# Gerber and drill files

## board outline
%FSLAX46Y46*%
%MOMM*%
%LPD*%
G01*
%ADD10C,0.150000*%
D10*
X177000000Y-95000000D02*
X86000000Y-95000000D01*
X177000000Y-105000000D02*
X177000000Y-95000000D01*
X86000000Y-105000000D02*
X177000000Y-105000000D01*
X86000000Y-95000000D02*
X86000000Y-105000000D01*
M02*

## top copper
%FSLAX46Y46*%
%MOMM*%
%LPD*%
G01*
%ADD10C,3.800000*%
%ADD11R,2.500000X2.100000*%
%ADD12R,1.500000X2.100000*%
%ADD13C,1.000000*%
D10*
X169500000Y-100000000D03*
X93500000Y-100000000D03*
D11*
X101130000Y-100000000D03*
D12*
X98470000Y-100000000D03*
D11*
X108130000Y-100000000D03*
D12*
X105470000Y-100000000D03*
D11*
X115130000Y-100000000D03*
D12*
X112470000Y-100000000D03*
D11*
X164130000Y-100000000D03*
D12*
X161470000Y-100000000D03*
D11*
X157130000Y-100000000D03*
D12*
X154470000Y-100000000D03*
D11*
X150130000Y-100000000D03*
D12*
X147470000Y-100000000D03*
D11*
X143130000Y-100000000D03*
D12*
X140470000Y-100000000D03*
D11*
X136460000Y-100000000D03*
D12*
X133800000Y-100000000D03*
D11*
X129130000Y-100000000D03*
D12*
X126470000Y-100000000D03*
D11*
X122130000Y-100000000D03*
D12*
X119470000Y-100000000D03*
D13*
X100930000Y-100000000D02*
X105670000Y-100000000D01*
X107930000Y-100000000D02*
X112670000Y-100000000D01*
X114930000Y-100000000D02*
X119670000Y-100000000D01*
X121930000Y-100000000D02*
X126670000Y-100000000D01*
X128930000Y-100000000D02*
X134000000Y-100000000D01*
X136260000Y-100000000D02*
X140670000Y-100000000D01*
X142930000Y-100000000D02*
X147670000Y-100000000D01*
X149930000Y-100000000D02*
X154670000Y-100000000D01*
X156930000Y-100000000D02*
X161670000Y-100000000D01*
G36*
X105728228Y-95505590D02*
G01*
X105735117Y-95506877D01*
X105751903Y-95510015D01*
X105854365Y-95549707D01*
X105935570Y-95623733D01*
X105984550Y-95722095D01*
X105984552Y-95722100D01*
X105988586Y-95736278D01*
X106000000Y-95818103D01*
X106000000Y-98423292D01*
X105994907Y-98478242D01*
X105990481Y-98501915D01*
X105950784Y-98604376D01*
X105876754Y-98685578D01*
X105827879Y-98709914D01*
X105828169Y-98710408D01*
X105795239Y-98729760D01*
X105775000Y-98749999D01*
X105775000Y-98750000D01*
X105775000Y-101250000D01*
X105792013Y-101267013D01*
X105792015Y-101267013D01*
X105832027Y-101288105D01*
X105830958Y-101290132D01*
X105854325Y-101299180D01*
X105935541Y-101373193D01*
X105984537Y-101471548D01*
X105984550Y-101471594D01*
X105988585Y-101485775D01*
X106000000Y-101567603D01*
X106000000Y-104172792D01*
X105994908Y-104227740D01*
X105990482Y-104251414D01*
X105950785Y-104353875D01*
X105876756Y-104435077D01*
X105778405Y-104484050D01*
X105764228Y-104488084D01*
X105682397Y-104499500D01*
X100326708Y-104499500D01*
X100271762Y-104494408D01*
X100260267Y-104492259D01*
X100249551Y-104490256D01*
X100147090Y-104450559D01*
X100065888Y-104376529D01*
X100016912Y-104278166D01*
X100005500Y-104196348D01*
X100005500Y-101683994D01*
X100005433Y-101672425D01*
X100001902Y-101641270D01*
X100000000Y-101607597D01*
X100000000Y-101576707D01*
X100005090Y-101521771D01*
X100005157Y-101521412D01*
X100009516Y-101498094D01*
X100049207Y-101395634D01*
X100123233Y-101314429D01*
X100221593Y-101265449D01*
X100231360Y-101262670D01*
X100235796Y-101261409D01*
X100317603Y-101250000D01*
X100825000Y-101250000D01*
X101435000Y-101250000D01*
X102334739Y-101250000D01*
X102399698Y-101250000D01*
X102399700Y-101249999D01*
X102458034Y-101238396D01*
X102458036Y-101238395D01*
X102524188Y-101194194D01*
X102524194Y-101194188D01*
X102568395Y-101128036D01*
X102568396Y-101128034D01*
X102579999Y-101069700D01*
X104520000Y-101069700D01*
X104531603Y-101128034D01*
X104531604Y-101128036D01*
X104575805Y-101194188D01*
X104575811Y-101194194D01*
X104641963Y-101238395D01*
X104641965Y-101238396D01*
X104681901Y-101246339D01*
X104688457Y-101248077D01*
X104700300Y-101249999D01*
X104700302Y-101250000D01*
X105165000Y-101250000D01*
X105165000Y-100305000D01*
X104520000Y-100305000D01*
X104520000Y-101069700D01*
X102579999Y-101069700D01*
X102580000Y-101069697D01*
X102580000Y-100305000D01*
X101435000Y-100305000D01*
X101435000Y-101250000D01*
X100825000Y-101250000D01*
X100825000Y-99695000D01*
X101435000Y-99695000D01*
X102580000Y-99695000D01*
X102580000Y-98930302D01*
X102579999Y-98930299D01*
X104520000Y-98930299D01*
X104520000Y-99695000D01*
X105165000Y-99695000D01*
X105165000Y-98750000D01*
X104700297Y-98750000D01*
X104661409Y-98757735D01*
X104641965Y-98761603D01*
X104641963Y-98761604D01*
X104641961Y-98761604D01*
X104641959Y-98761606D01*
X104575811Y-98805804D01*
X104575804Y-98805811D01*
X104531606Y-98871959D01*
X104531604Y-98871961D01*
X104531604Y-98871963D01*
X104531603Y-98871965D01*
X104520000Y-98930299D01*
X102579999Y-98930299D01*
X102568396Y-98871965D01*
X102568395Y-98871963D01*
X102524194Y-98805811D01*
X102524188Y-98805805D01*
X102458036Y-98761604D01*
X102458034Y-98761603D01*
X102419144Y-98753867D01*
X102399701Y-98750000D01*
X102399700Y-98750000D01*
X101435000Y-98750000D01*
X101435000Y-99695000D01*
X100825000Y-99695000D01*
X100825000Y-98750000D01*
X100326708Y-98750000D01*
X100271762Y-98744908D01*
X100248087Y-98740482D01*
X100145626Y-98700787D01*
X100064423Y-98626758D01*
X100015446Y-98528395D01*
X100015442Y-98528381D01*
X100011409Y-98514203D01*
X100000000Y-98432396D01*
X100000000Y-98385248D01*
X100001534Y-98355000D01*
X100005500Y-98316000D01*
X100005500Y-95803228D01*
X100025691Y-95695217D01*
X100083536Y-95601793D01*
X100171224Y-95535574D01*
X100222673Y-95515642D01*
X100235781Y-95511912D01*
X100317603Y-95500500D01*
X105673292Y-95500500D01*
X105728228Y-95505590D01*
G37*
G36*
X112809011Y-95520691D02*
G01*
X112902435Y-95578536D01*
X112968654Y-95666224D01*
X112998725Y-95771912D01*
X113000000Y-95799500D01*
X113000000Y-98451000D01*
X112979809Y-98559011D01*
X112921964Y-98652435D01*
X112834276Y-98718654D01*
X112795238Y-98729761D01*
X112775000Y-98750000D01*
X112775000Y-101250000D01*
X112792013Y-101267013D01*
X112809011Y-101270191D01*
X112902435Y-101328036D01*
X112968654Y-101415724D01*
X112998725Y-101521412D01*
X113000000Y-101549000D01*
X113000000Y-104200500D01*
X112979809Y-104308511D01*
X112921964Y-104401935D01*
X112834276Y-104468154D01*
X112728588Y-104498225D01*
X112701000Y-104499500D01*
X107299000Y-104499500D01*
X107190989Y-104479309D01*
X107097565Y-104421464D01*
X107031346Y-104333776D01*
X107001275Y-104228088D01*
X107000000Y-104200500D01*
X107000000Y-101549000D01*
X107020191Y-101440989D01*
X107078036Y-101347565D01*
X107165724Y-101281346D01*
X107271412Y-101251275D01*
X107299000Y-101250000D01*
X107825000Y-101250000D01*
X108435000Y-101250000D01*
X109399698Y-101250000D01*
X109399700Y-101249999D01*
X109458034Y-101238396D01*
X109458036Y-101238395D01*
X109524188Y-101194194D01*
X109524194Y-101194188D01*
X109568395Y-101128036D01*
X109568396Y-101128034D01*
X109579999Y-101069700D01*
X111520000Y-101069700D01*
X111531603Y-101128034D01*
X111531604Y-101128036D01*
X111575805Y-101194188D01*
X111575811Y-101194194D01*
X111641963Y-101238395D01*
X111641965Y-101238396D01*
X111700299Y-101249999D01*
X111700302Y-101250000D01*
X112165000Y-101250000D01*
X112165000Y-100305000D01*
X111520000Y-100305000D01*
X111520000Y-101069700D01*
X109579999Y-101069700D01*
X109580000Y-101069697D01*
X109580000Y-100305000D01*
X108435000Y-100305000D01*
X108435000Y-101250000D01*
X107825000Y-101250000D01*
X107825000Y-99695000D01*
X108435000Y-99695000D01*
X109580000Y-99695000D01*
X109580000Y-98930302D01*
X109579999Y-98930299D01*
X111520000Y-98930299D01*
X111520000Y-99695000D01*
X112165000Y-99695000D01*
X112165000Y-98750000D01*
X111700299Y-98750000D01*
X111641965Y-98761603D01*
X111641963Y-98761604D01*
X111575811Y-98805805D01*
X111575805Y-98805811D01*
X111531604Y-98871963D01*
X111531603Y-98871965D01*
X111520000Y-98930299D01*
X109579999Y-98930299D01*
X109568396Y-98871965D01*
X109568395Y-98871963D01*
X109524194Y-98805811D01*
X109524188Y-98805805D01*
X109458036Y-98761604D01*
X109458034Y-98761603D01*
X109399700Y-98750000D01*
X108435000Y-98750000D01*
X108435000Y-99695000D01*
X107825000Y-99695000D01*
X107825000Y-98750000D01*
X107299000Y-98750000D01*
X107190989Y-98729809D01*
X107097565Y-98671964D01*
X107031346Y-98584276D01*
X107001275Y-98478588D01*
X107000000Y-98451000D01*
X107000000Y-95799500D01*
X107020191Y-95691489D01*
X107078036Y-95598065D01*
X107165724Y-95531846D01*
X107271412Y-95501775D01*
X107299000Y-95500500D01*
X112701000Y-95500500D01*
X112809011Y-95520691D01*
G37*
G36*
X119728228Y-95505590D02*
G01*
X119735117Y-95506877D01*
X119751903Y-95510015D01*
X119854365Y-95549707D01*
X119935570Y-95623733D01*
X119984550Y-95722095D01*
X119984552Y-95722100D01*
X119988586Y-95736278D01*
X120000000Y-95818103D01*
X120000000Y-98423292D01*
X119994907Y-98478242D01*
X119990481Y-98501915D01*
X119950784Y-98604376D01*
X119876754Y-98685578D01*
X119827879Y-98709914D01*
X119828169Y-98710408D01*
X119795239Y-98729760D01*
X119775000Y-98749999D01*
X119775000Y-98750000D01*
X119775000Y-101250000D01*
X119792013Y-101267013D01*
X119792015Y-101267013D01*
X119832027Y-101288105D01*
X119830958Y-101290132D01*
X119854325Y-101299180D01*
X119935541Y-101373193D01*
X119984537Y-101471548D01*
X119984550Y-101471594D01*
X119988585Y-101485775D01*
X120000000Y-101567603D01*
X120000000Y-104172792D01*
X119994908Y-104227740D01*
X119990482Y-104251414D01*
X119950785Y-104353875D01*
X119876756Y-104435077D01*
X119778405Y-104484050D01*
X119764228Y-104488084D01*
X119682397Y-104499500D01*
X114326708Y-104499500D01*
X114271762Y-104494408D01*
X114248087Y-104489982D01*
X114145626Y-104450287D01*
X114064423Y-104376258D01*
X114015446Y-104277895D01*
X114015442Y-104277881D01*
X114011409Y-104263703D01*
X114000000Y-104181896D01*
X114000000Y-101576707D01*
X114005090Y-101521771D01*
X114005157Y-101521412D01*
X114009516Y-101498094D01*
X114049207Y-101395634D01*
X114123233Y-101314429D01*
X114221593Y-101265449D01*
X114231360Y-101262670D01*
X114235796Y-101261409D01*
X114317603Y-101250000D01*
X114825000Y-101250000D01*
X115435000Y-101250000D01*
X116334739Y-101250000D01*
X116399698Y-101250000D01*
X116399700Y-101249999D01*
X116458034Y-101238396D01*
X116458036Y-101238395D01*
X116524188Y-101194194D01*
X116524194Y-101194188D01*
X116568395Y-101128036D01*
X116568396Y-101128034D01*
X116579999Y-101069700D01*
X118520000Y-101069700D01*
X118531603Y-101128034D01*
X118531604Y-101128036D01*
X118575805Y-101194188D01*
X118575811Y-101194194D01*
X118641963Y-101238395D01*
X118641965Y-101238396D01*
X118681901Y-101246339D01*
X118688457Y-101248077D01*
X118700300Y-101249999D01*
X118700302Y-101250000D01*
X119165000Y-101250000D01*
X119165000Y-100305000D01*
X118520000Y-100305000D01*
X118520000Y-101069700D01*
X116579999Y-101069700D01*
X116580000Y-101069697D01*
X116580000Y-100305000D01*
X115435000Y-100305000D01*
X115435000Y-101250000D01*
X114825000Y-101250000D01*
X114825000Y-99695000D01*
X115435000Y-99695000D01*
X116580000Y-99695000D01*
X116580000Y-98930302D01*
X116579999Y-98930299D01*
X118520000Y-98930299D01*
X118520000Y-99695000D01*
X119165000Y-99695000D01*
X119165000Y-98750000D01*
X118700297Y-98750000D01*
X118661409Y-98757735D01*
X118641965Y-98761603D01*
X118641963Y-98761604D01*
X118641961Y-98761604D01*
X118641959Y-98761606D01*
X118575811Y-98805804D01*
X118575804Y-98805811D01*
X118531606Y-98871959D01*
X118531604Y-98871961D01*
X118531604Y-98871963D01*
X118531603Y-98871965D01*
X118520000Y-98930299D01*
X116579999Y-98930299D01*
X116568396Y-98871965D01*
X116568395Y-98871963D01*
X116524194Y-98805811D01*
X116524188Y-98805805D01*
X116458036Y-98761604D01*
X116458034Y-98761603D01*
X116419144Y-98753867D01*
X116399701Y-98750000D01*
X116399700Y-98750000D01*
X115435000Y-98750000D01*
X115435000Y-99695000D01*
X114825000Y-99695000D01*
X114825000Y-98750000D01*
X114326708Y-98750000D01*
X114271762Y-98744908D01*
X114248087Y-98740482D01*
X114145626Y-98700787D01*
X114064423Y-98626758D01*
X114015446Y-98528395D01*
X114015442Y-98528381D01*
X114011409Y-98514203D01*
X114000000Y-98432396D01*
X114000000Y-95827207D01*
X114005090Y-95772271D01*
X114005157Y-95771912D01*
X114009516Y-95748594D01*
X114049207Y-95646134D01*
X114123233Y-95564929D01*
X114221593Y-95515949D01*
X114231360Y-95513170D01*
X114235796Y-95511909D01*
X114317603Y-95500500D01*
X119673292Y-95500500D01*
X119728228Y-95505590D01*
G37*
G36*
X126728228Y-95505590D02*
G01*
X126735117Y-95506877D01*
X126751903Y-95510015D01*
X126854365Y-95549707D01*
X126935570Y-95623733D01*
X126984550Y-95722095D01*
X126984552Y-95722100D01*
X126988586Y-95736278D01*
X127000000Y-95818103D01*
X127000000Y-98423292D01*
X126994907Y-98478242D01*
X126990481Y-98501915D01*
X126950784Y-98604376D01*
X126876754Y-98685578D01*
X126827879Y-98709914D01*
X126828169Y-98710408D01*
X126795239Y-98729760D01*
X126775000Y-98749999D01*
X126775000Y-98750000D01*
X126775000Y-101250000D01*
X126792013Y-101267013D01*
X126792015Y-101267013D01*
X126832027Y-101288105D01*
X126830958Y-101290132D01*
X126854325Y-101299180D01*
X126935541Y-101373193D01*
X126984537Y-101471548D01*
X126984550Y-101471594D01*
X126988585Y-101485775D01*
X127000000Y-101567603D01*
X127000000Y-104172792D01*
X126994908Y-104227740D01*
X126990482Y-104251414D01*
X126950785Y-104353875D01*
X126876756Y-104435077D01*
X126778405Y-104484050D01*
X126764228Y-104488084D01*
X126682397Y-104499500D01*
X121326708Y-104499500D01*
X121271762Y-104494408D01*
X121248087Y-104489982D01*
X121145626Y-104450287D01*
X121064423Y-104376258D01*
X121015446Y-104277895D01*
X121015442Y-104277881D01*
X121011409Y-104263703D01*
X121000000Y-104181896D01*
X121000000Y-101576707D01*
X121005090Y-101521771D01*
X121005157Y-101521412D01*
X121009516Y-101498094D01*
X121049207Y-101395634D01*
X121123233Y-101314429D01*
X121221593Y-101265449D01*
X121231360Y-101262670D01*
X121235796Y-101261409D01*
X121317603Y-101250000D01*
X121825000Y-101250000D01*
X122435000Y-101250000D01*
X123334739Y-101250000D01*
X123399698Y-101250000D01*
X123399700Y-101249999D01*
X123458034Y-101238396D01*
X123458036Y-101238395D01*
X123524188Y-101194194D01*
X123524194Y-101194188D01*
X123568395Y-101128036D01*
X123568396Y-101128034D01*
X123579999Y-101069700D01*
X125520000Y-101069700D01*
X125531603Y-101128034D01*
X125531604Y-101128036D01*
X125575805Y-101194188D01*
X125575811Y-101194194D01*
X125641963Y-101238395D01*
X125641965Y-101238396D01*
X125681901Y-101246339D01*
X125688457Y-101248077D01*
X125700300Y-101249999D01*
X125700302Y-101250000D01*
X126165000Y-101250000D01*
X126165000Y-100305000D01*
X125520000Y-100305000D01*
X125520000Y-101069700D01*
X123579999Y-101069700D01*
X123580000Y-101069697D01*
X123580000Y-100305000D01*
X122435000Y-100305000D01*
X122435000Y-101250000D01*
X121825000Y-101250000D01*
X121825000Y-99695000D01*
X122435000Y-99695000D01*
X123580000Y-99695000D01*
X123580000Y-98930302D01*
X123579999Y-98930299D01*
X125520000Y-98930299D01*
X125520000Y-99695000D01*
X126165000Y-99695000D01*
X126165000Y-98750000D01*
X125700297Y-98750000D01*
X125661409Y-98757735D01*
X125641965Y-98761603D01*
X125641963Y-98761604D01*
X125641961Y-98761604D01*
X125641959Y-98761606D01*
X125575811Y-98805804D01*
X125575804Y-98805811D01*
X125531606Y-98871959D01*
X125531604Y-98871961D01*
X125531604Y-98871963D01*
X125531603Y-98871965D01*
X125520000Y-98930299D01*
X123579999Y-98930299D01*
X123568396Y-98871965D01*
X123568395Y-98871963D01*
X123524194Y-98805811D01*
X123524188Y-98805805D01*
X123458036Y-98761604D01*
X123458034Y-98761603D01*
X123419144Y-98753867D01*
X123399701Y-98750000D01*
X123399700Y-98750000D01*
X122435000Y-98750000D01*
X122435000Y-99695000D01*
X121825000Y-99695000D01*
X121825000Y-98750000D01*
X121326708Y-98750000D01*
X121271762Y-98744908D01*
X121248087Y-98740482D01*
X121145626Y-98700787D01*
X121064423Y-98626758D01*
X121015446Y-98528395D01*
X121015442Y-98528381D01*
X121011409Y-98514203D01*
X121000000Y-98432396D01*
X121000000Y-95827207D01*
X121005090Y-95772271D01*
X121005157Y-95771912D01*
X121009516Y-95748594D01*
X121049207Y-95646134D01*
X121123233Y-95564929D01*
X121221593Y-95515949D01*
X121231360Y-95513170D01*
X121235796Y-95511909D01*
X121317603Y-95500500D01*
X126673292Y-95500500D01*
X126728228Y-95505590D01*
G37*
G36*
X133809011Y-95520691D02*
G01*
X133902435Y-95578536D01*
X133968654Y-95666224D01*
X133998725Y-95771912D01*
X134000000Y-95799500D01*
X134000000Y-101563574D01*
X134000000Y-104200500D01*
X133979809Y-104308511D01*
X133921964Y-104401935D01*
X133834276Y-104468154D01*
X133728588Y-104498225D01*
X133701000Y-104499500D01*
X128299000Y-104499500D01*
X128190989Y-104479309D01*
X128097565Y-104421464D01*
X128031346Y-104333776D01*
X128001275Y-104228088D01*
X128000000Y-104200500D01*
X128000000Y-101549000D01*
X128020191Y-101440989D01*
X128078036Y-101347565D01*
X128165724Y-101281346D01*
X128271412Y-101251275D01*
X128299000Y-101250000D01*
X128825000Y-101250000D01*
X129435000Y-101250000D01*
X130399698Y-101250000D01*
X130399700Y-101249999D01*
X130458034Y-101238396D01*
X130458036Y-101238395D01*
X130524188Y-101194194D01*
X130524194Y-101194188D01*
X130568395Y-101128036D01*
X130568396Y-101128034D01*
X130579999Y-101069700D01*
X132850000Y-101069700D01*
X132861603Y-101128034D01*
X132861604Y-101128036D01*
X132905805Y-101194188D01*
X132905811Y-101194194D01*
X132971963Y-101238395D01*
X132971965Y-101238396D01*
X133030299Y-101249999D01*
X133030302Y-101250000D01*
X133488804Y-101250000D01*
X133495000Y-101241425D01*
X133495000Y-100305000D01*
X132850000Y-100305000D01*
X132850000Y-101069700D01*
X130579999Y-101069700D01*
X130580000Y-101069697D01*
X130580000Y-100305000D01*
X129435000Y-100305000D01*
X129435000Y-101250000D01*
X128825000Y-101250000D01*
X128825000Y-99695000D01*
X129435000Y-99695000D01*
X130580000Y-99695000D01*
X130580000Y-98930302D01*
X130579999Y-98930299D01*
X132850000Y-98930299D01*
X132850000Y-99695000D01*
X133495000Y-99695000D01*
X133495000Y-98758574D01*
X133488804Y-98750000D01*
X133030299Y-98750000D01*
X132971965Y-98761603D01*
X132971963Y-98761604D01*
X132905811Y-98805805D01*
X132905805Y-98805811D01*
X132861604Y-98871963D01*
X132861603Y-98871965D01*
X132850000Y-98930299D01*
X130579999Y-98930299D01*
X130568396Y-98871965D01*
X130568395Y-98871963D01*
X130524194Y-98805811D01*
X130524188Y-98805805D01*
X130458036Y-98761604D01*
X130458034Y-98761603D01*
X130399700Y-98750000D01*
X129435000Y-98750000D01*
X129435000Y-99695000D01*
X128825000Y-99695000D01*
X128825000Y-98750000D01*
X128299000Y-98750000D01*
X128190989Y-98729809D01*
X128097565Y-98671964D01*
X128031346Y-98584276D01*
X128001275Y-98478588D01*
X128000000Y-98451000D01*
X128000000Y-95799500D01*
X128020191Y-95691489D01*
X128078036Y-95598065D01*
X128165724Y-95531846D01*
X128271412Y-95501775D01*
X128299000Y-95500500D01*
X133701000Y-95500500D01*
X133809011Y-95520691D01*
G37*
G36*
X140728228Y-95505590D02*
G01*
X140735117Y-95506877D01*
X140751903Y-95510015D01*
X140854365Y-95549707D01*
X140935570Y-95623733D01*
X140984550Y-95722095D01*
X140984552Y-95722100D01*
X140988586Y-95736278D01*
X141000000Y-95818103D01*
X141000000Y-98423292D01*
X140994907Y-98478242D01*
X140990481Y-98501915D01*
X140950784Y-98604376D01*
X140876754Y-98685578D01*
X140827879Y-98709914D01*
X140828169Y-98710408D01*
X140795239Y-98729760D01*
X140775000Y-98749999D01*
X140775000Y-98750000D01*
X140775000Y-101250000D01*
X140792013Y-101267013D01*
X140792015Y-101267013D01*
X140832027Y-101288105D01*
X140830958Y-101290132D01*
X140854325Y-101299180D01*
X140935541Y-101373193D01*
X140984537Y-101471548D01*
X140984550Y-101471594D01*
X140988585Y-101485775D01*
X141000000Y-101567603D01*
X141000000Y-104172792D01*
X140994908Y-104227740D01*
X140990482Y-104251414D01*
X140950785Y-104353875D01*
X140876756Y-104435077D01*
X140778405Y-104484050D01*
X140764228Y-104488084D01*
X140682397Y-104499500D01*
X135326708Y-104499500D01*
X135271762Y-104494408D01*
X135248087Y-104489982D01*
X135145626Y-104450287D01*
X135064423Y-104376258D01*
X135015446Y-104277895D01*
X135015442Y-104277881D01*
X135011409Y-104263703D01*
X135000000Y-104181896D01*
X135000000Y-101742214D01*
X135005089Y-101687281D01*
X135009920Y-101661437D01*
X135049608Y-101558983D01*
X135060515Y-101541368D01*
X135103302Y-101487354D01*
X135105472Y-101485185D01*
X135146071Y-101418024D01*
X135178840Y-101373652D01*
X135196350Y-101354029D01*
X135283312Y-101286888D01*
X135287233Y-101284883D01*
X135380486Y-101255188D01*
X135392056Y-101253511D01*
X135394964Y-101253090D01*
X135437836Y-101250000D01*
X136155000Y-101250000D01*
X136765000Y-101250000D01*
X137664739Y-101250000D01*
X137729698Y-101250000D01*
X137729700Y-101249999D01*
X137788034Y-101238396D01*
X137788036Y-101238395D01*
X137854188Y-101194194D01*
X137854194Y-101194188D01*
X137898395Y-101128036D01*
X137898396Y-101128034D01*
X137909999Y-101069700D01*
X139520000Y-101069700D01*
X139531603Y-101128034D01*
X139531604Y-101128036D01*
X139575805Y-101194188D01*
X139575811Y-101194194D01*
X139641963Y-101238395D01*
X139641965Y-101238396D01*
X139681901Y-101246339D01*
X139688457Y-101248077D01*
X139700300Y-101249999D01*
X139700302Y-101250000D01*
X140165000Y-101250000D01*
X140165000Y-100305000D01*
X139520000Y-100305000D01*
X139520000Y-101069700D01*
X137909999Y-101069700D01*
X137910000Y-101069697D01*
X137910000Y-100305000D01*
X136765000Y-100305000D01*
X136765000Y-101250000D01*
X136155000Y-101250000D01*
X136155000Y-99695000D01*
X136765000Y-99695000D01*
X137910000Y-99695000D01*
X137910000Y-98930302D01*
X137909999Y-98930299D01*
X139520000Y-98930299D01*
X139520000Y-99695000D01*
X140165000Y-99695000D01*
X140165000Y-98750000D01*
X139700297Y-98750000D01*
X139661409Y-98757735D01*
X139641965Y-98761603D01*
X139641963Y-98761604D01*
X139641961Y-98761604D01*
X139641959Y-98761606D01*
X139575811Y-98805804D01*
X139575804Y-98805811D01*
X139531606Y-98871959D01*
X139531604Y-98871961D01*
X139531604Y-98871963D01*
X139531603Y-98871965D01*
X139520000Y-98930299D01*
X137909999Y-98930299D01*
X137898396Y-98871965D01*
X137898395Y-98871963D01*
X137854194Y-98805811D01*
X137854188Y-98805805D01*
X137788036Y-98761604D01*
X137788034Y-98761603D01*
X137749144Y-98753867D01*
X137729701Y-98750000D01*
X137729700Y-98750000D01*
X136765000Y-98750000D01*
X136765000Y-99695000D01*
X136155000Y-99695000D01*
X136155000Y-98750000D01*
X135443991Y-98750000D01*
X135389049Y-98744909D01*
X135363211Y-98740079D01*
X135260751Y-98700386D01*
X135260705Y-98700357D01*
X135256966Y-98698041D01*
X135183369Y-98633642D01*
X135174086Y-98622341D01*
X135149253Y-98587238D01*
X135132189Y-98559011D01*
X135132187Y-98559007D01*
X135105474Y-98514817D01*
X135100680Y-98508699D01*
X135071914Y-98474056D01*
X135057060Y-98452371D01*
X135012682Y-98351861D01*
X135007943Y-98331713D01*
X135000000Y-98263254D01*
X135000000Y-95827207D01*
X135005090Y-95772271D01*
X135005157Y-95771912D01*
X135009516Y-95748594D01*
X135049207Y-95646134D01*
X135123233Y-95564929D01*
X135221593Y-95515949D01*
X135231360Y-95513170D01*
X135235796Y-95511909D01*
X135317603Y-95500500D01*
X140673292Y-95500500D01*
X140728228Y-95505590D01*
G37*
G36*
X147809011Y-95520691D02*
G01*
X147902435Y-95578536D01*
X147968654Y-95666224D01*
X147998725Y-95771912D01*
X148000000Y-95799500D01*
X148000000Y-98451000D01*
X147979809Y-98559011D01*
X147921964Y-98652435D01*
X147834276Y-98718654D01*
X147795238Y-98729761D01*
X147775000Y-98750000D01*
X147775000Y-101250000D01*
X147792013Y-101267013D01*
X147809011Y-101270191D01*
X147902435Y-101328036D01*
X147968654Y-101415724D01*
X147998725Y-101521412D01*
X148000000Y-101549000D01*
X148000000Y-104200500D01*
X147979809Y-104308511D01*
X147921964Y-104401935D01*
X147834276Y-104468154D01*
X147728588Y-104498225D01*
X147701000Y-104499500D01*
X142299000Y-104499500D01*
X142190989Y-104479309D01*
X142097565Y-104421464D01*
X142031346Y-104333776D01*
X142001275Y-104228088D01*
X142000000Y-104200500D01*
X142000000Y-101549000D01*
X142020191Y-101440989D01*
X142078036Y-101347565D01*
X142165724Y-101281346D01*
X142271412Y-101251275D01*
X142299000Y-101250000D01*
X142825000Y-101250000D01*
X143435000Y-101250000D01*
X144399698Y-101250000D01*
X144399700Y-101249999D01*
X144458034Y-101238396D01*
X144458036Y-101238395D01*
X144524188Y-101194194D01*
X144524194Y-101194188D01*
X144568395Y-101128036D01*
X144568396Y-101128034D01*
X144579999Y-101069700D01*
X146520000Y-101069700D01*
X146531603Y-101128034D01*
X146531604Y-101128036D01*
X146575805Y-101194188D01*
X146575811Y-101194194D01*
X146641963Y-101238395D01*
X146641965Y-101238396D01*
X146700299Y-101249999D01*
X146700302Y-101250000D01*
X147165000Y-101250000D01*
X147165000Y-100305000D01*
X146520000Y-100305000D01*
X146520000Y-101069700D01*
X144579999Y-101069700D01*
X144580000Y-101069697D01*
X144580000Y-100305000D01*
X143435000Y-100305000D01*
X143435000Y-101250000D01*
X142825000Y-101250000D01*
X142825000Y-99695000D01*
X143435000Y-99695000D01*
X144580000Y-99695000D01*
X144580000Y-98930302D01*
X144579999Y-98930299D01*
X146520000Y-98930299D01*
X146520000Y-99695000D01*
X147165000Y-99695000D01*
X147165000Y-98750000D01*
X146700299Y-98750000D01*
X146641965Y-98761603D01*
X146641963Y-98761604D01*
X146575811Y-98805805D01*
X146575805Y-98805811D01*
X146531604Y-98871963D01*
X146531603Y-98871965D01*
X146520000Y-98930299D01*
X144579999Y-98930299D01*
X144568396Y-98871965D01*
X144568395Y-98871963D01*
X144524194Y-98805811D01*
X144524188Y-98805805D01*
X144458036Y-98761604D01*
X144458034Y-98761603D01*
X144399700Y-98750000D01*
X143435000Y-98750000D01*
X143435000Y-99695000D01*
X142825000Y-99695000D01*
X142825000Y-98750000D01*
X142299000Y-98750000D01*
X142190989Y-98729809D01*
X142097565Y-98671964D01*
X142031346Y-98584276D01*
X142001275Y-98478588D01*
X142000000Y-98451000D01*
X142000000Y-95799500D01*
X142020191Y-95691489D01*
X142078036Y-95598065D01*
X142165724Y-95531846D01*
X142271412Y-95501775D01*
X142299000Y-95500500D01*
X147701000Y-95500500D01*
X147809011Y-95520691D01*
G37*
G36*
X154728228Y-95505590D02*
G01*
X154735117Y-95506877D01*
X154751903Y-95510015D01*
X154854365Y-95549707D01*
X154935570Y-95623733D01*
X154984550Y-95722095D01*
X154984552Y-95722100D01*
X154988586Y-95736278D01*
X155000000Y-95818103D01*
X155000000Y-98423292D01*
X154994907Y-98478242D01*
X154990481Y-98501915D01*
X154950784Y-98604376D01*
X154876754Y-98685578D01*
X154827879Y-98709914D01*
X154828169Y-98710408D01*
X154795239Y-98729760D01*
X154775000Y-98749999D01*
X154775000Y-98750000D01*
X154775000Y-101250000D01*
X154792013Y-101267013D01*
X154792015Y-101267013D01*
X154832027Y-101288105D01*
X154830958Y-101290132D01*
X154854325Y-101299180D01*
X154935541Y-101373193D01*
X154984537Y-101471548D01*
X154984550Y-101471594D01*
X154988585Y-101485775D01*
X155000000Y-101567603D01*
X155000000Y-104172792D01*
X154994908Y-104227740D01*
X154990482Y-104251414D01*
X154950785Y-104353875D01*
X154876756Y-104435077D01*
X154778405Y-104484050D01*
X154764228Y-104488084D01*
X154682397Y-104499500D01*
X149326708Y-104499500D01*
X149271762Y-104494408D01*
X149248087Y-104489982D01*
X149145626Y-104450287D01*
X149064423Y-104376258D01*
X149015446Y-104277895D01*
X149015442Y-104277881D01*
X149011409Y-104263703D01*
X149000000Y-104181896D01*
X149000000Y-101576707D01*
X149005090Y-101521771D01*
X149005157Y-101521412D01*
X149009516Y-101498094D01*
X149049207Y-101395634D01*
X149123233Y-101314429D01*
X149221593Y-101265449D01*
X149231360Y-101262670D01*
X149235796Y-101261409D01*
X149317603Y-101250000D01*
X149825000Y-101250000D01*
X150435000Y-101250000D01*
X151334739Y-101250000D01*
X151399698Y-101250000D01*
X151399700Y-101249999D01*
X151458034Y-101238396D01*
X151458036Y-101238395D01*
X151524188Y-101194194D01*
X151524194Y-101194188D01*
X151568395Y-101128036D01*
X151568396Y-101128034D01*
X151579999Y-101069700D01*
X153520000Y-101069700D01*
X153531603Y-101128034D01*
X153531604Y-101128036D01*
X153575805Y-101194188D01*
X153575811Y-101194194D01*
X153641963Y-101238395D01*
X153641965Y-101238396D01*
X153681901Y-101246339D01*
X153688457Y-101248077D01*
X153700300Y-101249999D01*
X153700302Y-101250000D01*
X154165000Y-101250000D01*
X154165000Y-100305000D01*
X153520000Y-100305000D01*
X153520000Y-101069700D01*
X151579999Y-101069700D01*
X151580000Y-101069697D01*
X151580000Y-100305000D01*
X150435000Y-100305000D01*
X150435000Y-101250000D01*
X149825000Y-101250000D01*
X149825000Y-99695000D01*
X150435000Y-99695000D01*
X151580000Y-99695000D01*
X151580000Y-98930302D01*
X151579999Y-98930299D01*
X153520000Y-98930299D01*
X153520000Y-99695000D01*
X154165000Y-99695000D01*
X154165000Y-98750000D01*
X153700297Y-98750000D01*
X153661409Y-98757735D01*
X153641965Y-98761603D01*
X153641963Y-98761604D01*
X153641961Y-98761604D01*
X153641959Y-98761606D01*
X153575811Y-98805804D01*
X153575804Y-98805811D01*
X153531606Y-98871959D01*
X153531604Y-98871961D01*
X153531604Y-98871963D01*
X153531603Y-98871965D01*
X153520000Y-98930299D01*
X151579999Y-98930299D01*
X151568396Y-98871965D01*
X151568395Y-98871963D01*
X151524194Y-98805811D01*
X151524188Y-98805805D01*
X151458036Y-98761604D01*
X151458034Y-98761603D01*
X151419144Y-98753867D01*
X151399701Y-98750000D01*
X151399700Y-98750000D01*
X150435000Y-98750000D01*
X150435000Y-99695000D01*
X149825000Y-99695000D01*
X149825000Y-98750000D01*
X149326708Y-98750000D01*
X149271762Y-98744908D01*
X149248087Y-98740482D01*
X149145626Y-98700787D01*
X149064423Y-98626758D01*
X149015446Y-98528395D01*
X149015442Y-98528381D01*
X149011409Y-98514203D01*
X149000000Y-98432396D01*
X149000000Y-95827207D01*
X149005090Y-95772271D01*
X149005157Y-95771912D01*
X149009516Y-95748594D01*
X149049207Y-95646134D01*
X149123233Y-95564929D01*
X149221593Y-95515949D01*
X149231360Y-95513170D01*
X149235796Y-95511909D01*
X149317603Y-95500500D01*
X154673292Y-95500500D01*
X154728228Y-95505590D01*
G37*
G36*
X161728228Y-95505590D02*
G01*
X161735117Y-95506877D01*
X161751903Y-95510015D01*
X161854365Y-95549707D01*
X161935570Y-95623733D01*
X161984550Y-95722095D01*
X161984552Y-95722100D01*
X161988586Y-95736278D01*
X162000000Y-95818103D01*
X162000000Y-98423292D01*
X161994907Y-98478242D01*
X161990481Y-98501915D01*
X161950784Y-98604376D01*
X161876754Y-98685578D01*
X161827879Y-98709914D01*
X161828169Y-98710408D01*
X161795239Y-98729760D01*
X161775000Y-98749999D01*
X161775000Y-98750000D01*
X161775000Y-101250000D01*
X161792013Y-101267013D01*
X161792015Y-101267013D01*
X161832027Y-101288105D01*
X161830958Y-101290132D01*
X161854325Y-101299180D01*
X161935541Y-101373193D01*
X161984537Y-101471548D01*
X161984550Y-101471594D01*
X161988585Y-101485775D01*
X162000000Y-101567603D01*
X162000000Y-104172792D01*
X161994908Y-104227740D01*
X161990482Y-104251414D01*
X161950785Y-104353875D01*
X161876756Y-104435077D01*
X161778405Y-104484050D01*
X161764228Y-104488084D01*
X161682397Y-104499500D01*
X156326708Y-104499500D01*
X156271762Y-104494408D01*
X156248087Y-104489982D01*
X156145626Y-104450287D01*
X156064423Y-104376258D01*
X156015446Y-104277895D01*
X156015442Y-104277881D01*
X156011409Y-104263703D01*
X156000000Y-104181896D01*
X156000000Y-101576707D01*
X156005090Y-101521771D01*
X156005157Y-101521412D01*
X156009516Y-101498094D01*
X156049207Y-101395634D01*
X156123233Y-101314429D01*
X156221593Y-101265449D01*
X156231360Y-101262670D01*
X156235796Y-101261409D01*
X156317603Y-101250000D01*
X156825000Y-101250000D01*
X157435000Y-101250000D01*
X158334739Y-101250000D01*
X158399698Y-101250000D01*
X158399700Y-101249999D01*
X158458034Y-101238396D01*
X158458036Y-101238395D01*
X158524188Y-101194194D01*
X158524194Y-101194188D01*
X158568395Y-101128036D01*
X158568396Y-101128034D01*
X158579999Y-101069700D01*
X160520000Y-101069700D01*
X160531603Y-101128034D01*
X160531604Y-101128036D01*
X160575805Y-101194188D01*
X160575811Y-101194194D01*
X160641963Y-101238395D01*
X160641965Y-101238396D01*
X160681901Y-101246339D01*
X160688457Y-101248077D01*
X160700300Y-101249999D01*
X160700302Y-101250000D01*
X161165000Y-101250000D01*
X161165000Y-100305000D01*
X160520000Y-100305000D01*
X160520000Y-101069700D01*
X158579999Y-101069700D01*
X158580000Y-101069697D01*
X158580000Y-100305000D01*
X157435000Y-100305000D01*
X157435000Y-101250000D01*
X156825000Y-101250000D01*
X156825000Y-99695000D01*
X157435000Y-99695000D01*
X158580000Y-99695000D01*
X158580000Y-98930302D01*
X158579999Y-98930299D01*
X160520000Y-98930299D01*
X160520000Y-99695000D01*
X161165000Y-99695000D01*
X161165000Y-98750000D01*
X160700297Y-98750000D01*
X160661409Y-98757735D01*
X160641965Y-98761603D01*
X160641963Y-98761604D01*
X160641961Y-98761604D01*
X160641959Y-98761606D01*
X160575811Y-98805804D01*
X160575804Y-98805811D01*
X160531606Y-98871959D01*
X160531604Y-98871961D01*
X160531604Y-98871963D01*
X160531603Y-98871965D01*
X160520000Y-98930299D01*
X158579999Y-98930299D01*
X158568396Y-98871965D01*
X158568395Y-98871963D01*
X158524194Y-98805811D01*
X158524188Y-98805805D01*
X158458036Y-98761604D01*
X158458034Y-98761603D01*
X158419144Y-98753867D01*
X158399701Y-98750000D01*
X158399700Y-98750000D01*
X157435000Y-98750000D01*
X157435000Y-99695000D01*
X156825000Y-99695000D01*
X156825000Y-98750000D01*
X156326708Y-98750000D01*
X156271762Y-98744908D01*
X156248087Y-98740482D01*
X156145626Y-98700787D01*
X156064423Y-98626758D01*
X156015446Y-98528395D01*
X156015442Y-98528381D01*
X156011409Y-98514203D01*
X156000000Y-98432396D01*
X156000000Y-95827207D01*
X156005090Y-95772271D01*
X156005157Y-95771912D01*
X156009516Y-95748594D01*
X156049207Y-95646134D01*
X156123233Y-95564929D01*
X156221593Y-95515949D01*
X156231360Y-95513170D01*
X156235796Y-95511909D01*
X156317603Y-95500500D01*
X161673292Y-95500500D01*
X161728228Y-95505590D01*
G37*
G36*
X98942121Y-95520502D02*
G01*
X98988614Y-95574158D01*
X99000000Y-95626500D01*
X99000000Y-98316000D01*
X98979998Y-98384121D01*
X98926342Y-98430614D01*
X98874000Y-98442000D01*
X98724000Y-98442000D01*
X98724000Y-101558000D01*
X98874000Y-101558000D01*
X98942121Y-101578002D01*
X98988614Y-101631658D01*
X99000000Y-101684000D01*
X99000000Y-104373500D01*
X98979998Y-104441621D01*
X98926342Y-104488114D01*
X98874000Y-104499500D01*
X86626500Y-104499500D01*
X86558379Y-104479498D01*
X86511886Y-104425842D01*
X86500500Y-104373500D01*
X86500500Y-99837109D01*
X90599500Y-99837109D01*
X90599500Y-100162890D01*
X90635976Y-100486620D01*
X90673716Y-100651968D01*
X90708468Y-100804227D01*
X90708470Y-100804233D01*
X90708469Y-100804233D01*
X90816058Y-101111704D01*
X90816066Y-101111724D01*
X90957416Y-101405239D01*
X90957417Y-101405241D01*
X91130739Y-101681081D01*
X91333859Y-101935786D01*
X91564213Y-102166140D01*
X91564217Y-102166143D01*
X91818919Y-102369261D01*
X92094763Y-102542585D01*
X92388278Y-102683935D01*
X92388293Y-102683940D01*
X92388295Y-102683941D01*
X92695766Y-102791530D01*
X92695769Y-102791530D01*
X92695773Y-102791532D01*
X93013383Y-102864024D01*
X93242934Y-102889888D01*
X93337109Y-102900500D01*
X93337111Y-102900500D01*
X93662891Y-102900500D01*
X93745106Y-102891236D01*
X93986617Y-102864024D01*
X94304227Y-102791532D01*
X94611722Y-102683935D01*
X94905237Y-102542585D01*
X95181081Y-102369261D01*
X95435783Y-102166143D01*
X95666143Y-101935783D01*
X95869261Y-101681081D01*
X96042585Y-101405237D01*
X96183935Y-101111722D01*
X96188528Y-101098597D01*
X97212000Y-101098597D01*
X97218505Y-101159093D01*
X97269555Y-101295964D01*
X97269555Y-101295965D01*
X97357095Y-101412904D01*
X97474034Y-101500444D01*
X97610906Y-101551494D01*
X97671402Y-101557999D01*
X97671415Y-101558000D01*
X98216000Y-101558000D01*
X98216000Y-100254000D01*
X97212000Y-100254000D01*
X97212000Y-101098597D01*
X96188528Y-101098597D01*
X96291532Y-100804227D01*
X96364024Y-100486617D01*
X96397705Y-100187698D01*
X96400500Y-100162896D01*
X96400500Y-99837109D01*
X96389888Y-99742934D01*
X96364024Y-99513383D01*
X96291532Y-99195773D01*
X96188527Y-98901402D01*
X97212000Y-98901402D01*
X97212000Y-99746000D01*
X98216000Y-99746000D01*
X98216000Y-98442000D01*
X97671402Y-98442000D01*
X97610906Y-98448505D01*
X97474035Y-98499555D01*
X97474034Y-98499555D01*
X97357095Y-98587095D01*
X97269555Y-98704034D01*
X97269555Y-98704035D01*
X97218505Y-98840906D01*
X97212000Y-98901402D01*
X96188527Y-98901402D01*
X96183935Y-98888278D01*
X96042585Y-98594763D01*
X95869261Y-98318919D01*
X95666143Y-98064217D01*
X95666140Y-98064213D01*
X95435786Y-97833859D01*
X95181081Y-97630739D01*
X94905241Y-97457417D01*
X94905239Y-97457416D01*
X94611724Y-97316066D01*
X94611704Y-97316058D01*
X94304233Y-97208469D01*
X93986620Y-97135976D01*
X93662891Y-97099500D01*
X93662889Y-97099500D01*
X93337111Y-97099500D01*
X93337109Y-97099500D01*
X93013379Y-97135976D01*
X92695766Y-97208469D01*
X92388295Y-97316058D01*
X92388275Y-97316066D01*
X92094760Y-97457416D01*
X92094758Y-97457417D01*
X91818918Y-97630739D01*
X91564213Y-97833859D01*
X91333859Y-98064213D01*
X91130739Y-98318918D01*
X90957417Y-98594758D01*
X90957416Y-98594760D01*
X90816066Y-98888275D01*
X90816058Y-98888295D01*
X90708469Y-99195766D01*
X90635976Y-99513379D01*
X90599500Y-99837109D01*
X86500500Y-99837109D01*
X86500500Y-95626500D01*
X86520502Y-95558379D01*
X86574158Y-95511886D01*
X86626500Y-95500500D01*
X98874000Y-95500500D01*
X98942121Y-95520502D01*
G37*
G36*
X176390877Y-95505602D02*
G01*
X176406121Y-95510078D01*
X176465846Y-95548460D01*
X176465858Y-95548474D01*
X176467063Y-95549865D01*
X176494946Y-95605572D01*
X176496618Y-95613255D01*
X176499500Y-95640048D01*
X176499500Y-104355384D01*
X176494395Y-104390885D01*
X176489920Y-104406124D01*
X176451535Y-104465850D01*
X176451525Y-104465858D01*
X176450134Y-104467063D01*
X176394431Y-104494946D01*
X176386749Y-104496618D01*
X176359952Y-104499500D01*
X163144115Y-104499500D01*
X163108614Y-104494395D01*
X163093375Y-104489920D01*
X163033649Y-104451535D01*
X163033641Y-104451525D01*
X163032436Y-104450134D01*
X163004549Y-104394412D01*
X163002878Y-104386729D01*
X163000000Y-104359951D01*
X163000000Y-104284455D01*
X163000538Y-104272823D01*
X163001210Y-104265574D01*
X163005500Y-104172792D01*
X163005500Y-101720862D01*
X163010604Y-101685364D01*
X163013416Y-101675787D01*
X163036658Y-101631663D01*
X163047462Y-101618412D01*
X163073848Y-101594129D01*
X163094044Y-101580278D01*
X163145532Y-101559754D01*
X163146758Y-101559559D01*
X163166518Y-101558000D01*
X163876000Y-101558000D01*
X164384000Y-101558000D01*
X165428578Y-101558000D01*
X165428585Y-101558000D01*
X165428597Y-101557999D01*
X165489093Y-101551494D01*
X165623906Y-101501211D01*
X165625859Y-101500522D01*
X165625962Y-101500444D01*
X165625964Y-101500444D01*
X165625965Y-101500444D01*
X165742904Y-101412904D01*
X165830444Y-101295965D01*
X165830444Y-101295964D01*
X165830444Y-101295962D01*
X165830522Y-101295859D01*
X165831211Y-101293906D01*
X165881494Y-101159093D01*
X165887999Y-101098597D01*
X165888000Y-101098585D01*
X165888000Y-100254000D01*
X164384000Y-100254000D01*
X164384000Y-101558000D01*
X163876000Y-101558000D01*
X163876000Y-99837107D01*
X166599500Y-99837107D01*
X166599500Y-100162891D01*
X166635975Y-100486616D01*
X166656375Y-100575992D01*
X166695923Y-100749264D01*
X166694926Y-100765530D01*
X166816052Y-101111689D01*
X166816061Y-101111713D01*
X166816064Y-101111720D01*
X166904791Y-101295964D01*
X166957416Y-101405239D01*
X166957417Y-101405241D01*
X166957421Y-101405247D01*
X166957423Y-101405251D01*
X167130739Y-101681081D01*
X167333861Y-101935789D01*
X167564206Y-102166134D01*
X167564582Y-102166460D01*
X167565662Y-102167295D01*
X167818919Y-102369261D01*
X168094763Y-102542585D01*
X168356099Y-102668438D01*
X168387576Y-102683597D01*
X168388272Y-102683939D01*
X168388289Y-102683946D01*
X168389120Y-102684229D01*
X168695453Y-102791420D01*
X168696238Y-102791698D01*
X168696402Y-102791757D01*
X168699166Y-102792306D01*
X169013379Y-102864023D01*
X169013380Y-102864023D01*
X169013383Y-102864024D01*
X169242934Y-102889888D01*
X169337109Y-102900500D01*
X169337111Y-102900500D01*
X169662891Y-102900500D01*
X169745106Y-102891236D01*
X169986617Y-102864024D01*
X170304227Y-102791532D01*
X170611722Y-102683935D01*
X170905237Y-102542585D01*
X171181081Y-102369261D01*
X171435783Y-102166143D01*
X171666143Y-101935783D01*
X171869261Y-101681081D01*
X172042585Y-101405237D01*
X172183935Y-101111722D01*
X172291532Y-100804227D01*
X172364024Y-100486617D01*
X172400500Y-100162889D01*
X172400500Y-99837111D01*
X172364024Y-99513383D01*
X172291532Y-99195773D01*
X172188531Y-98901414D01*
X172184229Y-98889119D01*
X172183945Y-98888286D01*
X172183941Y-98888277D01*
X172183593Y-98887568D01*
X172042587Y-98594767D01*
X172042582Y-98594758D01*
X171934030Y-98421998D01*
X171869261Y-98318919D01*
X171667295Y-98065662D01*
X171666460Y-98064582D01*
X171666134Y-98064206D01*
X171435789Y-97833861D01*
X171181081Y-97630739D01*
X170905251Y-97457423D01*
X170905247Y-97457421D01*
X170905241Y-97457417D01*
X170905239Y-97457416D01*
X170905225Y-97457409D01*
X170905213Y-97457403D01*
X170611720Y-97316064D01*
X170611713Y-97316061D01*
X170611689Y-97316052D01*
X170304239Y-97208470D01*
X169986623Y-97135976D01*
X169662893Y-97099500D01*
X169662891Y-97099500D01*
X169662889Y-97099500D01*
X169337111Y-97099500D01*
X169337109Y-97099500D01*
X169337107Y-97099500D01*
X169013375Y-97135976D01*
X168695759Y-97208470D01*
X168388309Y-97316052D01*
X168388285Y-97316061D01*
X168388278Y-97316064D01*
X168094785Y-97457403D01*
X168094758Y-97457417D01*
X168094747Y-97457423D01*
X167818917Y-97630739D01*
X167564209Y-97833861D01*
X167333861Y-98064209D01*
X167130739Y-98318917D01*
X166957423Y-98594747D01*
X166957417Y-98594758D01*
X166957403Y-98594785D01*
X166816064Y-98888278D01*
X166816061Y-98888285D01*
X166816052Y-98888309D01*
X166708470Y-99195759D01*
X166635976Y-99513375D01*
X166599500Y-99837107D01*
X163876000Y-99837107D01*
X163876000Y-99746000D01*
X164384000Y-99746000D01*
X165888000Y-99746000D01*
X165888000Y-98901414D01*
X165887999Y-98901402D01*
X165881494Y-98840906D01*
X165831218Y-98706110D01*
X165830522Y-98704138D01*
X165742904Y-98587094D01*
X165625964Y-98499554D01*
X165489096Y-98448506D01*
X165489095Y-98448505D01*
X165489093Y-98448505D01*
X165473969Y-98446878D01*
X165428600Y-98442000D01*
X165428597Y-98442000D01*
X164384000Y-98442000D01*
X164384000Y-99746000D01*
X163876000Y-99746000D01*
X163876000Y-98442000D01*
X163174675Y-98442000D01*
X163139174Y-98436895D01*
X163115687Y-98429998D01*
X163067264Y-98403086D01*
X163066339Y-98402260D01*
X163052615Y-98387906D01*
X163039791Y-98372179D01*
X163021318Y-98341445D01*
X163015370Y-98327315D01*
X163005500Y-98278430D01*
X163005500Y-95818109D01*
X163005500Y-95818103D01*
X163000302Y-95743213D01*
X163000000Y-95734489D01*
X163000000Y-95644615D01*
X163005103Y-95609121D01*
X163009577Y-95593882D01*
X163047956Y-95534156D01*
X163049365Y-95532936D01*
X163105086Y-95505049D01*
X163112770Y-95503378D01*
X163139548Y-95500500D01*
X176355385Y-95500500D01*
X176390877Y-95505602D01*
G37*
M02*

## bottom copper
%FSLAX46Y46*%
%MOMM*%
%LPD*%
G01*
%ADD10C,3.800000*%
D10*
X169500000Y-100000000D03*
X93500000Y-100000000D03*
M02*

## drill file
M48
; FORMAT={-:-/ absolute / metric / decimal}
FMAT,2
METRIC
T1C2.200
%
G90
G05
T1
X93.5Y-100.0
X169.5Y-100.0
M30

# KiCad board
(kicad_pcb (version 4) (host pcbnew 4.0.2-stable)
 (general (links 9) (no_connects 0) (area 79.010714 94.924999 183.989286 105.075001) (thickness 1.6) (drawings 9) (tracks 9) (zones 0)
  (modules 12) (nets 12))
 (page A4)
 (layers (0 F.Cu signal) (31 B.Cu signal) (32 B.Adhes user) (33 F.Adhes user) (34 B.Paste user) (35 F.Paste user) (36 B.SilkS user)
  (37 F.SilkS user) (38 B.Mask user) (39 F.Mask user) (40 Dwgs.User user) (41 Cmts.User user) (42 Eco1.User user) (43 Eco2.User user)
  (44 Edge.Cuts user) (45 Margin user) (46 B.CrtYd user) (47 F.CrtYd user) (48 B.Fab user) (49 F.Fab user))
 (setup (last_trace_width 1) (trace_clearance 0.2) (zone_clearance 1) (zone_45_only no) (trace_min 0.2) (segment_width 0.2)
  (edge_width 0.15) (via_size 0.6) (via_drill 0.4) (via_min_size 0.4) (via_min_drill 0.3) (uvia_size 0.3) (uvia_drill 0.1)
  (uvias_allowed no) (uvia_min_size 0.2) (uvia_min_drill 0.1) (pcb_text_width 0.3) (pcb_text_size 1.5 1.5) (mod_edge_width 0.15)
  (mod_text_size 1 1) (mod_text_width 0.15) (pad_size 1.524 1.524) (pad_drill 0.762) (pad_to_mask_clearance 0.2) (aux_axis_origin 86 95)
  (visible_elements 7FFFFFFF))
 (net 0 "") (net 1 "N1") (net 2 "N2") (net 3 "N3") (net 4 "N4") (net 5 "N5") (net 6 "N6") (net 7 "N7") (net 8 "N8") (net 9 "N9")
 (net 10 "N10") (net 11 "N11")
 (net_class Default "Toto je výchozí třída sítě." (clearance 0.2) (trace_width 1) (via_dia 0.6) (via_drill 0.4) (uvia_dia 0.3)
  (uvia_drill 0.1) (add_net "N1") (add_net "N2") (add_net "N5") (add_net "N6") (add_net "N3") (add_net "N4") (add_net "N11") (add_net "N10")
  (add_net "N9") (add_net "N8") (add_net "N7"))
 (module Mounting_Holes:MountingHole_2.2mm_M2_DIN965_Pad (layer F.Cu) (at 169.5 100)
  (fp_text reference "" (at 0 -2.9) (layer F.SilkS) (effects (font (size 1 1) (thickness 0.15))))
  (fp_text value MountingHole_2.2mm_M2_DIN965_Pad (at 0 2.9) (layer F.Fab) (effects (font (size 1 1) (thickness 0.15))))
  (pad 1 thru_hole circle (at 0 0) (size 3.8 3.8) (drill 2.2) (layers *.Cu *.Mask F.SilkS)))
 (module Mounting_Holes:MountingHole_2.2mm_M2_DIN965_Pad (layer F.Cu) (at 93.5 100)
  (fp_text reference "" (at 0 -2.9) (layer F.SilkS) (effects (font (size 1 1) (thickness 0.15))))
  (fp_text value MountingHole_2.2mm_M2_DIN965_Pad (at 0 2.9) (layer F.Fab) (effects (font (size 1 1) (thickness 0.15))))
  (pad 1 thru_hole circle (at 0 0) (size 3.8 3.8) (drill 2.2) (layers *.Cu *.Mask F.SilkS)))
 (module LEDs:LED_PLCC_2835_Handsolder (layer F.Cu) (at 100 100)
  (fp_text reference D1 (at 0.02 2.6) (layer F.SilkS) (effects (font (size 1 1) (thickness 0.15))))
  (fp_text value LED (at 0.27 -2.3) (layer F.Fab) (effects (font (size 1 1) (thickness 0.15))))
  (pad 1 smd rect (at 1.13 0) (size 2.5 2.1) (layers F.Cu F.Paste F.Mask) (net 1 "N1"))
  (pad 2 smd rect (at -1.53 0) (size 1.5 2.1) (layers F.Cu F.Paste F.Mask) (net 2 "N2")))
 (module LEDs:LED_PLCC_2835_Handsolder (layer F.Cu) (at 107 100)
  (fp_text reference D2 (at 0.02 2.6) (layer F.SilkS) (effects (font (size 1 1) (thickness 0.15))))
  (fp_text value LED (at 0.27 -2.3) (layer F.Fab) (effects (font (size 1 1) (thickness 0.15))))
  (pad 1 smd rect (at 1.13 0) (size 2.5 2.1) (layers F.Cu F.Paste F.Mask) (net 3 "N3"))
  (pad 2 smd rect (at -1.53 0) (size 1.5 2.1) (layers F.Cu F.Paste F.Mask) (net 1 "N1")))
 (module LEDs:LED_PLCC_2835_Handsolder (layer F.Cu) (at 114 100)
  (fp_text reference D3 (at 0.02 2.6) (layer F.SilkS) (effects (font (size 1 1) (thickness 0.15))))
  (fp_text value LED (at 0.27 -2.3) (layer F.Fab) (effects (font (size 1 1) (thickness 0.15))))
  (pad 1 smd rect (at 1.13 0) (size 2.5 2.1) (layers F.Cu F.Paste F.Mask) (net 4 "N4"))
  (pad 2 smd rect (at -1.53 0) (size 1.5 2.1) (layers F.Cu F.Paste F.Mask) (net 3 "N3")))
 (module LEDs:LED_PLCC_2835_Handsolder (layer F.Cu) (at 163 100)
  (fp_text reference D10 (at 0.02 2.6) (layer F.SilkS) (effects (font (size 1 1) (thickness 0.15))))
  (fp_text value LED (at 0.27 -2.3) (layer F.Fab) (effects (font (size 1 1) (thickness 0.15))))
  (pad 1 smd rect (at 1.13 0) (size 2.5 2.1) (layers F.Cu F.Paste F.Mask) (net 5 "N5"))
  (pad 2 smd rect (at -1.53 0) (size 1.5 2.1) (layers F.Cu F.Paste F.Mask) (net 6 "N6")))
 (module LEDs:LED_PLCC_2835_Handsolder (layer F.Cu) (at 156 100)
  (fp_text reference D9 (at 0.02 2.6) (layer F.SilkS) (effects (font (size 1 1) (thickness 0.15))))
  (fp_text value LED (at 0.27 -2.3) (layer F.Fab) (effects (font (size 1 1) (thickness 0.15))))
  (pad 1 smd rect (at 1.13 0) (size 2.5 2.1) (layers F.Cu F.Paste F.Mask) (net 6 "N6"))
  (pad 2 smd rect (at -1.53 0) (size 1.5 2.1) (layers F.Cu F.Paste F.Mask) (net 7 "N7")))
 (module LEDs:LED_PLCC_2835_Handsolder (layer F.Cu) (at 149 100)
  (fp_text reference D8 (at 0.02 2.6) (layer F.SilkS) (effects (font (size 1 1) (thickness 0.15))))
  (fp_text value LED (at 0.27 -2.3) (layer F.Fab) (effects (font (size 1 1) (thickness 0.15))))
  (pad 1 smd rect (at 1.13 0) (size 2.5 2.1) (layers F.Cu F.Paste F.Mask) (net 7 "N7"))
  (pad 2 smd rect (at -1.53 0) (size 1.5 2.1) (layers F.Cu F.Paste F.Mask) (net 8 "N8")))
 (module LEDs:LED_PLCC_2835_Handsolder (layer F.Cu) (at 142 100)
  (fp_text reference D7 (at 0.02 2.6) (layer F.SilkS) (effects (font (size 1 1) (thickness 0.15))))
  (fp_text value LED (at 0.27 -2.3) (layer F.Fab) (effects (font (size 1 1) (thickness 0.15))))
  (pad 1 smd rect (at 1.13 0) (size 2.5 2.1) (layers F.Cu F.Paste F.Mask) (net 8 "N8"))
  (pad 2 smd rect (at -1.53 0) (size 1.5 2.1) (layers F.Cu F.Paste F.Mask) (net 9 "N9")))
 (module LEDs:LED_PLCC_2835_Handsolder (layer F.Cu) (at 135.33 100)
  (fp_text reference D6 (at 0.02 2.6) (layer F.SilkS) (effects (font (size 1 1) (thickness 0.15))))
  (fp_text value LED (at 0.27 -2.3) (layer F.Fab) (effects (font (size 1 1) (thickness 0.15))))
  (pad 1 smd rect (at 1.13 0) (size 2.5 2.1) (layers F.Cu F.Paste F.Mask) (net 9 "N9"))
  (pad 2 smd rect (at -1.53 0) (size 1.5 2.1) (layers F.Cu F.Paste F.Mask) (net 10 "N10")))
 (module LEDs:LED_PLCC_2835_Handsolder (layer F.Cu) (at 128 100)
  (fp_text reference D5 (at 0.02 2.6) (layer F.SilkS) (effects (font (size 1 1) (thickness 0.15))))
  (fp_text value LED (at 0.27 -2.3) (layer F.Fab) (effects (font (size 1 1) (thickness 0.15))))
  (pad 1 smd rect (at 1.13 0) (size 2.5 2.1) (layers F.Cu F.Paste F.Mask) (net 10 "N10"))
  (pad 2 smd rect (at -1.53 0) (size 1.5 2.1) (layers F.Cu F.Paste F.Mask) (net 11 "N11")))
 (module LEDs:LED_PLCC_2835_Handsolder (layer F.Cu) (at 121 100)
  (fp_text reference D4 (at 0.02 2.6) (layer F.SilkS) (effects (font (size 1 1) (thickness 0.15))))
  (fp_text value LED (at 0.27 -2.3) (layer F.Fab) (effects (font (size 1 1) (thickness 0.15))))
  (pad 1 smd rect (at 1.13 0) (size 2.5 2.1) (layers F.Cu F.Paste F.Mask) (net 11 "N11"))
  (pad 2 smd rect (at -1.53 0) (size 1.5 2.1) (layers F.Cu F.Paste F.Mask) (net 4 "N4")))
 (gr_line (start 177 95) (end 86 95) (layer Edge.Cuts) (width 0.15))
 (gr_line (start 177 105) (end 177 95) (layer Edge.Cuts) (width 0.15))
 (gr_line (start 86 105) (end 177 105) (layer Edge.Cuts) (width 0.15))
 (gr_line (start 86 95) (end 86 105) (layer Edge.Cuts) (width 0.15))
 (segment (start 100.93 100) (end 105.67 100) (width 1) (layer F.Cu) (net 1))
 (segment (start 107.93 100) (end 112.67 100) (width 1) (layer F.Cu) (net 3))
 (segment (start 114.93 100) (end 119.67 100) (width 1) (layer F.Cu) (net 4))
 (segment (start 121.93 100) (end 126.67 100) (width 1) (layer F.Cu) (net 11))
 (segment (start 128.93 100) (end 134 100) (width 1) (layer F.Cu) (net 10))
 (segment (start 136.26 100) (end 140.67 100) (width 1) (layer F.Cu) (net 9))
 (segment (start 142.93 100) (end 147.67 100) (width 1) (layer F.Cu) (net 8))
 (segment (start 149.93 100) (end 154.67 100) (width 1) (layer F.Cu) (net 7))
 (segment (start 156.93 100) (end 161.67 100) (width 1) (layer F.Cu) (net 6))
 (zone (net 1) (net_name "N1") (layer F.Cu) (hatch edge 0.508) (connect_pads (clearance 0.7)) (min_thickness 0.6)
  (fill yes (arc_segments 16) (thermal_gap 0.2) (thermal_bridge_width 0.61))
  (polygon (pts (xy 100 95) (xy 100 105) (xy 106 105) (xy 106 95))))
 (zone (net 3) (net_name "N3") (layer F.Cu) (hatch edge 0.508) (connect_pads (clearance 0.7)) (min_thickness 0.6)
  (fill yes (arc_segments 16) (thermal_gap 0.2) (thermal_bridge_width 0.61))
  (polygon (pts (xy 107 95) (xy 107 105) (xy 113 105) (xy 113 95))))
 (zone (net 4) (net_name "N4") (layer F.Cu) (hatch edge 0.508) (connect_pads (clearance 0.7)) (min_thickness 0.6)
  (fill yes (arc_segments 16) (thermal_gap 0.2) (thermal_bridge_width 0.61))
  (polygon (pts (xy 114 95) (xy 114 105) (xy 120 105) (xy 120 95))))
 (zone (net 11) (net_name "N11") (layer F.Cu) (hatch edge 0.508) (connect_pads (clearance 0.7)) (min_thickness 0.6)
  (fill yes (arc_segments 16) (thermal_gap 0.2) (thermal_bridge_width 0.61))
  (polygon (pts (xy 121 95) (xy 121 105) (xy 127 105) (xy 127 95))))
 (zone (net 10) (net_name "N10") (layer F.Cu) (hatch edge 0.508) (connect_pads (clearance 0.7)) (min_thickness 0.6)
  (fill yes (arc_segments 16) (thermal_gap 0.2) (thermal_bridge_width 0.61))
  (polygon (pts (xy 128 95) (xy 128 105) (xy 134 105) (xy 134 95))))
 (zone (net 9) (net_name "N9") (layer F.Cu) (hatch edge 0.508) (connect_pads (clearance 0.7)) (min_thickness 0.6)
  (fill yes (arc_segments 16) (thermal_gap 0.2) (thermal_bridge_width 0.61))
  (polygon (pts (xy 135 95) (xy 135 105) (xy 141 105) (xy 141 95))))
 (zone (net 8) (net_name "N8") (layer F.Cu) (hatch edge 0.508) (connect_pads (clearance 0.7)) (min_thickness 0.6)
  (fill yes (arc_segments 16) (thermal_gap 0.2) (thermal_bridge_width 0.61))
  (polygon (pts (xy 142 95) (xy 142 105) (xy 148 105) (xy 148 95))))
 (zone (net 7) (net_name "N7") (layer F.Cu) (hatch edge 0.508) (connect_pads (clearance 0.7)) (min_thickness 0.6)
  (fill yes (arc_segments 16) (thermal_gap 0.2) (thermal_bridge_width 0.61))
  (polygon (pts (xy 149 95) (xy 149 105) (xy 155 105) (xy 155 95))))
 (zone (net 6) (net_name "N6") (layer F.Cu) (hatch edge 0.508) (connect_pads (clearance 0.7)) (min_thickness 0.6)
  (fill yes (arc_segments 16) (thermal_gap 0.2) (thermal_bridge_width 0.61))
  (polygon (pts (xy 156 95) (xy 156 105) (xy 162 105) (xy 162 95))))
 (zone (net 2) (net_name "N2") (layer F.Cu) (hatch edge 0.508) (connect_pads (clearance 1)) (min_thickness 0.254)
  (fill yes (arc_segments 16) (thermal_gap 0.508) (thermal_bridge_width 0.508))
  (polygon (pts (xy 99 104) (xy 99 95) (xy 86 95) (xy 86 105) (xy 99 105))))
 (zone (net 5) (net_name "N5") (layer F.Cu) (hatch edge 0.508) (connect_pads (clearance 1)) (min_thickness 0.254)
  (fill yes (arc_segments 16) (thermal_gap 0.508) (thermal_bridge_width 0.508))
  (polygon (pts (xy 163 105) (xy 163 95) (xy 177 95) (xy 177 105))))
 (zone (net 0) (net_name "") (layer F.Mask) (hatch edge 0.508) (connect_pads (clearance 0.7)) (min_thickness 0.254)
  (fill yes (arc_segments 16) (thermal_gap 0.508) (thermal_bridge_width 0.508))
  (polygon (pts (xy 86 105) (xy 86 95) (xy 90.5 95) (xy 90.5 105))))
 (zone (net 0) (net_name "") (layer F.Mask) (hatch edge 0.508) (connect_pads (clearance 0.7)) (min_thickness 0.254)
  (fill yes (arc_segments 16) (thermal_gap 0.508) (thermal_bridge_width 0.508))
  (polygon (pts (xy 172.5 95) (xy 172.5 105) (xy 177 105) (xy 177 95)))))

